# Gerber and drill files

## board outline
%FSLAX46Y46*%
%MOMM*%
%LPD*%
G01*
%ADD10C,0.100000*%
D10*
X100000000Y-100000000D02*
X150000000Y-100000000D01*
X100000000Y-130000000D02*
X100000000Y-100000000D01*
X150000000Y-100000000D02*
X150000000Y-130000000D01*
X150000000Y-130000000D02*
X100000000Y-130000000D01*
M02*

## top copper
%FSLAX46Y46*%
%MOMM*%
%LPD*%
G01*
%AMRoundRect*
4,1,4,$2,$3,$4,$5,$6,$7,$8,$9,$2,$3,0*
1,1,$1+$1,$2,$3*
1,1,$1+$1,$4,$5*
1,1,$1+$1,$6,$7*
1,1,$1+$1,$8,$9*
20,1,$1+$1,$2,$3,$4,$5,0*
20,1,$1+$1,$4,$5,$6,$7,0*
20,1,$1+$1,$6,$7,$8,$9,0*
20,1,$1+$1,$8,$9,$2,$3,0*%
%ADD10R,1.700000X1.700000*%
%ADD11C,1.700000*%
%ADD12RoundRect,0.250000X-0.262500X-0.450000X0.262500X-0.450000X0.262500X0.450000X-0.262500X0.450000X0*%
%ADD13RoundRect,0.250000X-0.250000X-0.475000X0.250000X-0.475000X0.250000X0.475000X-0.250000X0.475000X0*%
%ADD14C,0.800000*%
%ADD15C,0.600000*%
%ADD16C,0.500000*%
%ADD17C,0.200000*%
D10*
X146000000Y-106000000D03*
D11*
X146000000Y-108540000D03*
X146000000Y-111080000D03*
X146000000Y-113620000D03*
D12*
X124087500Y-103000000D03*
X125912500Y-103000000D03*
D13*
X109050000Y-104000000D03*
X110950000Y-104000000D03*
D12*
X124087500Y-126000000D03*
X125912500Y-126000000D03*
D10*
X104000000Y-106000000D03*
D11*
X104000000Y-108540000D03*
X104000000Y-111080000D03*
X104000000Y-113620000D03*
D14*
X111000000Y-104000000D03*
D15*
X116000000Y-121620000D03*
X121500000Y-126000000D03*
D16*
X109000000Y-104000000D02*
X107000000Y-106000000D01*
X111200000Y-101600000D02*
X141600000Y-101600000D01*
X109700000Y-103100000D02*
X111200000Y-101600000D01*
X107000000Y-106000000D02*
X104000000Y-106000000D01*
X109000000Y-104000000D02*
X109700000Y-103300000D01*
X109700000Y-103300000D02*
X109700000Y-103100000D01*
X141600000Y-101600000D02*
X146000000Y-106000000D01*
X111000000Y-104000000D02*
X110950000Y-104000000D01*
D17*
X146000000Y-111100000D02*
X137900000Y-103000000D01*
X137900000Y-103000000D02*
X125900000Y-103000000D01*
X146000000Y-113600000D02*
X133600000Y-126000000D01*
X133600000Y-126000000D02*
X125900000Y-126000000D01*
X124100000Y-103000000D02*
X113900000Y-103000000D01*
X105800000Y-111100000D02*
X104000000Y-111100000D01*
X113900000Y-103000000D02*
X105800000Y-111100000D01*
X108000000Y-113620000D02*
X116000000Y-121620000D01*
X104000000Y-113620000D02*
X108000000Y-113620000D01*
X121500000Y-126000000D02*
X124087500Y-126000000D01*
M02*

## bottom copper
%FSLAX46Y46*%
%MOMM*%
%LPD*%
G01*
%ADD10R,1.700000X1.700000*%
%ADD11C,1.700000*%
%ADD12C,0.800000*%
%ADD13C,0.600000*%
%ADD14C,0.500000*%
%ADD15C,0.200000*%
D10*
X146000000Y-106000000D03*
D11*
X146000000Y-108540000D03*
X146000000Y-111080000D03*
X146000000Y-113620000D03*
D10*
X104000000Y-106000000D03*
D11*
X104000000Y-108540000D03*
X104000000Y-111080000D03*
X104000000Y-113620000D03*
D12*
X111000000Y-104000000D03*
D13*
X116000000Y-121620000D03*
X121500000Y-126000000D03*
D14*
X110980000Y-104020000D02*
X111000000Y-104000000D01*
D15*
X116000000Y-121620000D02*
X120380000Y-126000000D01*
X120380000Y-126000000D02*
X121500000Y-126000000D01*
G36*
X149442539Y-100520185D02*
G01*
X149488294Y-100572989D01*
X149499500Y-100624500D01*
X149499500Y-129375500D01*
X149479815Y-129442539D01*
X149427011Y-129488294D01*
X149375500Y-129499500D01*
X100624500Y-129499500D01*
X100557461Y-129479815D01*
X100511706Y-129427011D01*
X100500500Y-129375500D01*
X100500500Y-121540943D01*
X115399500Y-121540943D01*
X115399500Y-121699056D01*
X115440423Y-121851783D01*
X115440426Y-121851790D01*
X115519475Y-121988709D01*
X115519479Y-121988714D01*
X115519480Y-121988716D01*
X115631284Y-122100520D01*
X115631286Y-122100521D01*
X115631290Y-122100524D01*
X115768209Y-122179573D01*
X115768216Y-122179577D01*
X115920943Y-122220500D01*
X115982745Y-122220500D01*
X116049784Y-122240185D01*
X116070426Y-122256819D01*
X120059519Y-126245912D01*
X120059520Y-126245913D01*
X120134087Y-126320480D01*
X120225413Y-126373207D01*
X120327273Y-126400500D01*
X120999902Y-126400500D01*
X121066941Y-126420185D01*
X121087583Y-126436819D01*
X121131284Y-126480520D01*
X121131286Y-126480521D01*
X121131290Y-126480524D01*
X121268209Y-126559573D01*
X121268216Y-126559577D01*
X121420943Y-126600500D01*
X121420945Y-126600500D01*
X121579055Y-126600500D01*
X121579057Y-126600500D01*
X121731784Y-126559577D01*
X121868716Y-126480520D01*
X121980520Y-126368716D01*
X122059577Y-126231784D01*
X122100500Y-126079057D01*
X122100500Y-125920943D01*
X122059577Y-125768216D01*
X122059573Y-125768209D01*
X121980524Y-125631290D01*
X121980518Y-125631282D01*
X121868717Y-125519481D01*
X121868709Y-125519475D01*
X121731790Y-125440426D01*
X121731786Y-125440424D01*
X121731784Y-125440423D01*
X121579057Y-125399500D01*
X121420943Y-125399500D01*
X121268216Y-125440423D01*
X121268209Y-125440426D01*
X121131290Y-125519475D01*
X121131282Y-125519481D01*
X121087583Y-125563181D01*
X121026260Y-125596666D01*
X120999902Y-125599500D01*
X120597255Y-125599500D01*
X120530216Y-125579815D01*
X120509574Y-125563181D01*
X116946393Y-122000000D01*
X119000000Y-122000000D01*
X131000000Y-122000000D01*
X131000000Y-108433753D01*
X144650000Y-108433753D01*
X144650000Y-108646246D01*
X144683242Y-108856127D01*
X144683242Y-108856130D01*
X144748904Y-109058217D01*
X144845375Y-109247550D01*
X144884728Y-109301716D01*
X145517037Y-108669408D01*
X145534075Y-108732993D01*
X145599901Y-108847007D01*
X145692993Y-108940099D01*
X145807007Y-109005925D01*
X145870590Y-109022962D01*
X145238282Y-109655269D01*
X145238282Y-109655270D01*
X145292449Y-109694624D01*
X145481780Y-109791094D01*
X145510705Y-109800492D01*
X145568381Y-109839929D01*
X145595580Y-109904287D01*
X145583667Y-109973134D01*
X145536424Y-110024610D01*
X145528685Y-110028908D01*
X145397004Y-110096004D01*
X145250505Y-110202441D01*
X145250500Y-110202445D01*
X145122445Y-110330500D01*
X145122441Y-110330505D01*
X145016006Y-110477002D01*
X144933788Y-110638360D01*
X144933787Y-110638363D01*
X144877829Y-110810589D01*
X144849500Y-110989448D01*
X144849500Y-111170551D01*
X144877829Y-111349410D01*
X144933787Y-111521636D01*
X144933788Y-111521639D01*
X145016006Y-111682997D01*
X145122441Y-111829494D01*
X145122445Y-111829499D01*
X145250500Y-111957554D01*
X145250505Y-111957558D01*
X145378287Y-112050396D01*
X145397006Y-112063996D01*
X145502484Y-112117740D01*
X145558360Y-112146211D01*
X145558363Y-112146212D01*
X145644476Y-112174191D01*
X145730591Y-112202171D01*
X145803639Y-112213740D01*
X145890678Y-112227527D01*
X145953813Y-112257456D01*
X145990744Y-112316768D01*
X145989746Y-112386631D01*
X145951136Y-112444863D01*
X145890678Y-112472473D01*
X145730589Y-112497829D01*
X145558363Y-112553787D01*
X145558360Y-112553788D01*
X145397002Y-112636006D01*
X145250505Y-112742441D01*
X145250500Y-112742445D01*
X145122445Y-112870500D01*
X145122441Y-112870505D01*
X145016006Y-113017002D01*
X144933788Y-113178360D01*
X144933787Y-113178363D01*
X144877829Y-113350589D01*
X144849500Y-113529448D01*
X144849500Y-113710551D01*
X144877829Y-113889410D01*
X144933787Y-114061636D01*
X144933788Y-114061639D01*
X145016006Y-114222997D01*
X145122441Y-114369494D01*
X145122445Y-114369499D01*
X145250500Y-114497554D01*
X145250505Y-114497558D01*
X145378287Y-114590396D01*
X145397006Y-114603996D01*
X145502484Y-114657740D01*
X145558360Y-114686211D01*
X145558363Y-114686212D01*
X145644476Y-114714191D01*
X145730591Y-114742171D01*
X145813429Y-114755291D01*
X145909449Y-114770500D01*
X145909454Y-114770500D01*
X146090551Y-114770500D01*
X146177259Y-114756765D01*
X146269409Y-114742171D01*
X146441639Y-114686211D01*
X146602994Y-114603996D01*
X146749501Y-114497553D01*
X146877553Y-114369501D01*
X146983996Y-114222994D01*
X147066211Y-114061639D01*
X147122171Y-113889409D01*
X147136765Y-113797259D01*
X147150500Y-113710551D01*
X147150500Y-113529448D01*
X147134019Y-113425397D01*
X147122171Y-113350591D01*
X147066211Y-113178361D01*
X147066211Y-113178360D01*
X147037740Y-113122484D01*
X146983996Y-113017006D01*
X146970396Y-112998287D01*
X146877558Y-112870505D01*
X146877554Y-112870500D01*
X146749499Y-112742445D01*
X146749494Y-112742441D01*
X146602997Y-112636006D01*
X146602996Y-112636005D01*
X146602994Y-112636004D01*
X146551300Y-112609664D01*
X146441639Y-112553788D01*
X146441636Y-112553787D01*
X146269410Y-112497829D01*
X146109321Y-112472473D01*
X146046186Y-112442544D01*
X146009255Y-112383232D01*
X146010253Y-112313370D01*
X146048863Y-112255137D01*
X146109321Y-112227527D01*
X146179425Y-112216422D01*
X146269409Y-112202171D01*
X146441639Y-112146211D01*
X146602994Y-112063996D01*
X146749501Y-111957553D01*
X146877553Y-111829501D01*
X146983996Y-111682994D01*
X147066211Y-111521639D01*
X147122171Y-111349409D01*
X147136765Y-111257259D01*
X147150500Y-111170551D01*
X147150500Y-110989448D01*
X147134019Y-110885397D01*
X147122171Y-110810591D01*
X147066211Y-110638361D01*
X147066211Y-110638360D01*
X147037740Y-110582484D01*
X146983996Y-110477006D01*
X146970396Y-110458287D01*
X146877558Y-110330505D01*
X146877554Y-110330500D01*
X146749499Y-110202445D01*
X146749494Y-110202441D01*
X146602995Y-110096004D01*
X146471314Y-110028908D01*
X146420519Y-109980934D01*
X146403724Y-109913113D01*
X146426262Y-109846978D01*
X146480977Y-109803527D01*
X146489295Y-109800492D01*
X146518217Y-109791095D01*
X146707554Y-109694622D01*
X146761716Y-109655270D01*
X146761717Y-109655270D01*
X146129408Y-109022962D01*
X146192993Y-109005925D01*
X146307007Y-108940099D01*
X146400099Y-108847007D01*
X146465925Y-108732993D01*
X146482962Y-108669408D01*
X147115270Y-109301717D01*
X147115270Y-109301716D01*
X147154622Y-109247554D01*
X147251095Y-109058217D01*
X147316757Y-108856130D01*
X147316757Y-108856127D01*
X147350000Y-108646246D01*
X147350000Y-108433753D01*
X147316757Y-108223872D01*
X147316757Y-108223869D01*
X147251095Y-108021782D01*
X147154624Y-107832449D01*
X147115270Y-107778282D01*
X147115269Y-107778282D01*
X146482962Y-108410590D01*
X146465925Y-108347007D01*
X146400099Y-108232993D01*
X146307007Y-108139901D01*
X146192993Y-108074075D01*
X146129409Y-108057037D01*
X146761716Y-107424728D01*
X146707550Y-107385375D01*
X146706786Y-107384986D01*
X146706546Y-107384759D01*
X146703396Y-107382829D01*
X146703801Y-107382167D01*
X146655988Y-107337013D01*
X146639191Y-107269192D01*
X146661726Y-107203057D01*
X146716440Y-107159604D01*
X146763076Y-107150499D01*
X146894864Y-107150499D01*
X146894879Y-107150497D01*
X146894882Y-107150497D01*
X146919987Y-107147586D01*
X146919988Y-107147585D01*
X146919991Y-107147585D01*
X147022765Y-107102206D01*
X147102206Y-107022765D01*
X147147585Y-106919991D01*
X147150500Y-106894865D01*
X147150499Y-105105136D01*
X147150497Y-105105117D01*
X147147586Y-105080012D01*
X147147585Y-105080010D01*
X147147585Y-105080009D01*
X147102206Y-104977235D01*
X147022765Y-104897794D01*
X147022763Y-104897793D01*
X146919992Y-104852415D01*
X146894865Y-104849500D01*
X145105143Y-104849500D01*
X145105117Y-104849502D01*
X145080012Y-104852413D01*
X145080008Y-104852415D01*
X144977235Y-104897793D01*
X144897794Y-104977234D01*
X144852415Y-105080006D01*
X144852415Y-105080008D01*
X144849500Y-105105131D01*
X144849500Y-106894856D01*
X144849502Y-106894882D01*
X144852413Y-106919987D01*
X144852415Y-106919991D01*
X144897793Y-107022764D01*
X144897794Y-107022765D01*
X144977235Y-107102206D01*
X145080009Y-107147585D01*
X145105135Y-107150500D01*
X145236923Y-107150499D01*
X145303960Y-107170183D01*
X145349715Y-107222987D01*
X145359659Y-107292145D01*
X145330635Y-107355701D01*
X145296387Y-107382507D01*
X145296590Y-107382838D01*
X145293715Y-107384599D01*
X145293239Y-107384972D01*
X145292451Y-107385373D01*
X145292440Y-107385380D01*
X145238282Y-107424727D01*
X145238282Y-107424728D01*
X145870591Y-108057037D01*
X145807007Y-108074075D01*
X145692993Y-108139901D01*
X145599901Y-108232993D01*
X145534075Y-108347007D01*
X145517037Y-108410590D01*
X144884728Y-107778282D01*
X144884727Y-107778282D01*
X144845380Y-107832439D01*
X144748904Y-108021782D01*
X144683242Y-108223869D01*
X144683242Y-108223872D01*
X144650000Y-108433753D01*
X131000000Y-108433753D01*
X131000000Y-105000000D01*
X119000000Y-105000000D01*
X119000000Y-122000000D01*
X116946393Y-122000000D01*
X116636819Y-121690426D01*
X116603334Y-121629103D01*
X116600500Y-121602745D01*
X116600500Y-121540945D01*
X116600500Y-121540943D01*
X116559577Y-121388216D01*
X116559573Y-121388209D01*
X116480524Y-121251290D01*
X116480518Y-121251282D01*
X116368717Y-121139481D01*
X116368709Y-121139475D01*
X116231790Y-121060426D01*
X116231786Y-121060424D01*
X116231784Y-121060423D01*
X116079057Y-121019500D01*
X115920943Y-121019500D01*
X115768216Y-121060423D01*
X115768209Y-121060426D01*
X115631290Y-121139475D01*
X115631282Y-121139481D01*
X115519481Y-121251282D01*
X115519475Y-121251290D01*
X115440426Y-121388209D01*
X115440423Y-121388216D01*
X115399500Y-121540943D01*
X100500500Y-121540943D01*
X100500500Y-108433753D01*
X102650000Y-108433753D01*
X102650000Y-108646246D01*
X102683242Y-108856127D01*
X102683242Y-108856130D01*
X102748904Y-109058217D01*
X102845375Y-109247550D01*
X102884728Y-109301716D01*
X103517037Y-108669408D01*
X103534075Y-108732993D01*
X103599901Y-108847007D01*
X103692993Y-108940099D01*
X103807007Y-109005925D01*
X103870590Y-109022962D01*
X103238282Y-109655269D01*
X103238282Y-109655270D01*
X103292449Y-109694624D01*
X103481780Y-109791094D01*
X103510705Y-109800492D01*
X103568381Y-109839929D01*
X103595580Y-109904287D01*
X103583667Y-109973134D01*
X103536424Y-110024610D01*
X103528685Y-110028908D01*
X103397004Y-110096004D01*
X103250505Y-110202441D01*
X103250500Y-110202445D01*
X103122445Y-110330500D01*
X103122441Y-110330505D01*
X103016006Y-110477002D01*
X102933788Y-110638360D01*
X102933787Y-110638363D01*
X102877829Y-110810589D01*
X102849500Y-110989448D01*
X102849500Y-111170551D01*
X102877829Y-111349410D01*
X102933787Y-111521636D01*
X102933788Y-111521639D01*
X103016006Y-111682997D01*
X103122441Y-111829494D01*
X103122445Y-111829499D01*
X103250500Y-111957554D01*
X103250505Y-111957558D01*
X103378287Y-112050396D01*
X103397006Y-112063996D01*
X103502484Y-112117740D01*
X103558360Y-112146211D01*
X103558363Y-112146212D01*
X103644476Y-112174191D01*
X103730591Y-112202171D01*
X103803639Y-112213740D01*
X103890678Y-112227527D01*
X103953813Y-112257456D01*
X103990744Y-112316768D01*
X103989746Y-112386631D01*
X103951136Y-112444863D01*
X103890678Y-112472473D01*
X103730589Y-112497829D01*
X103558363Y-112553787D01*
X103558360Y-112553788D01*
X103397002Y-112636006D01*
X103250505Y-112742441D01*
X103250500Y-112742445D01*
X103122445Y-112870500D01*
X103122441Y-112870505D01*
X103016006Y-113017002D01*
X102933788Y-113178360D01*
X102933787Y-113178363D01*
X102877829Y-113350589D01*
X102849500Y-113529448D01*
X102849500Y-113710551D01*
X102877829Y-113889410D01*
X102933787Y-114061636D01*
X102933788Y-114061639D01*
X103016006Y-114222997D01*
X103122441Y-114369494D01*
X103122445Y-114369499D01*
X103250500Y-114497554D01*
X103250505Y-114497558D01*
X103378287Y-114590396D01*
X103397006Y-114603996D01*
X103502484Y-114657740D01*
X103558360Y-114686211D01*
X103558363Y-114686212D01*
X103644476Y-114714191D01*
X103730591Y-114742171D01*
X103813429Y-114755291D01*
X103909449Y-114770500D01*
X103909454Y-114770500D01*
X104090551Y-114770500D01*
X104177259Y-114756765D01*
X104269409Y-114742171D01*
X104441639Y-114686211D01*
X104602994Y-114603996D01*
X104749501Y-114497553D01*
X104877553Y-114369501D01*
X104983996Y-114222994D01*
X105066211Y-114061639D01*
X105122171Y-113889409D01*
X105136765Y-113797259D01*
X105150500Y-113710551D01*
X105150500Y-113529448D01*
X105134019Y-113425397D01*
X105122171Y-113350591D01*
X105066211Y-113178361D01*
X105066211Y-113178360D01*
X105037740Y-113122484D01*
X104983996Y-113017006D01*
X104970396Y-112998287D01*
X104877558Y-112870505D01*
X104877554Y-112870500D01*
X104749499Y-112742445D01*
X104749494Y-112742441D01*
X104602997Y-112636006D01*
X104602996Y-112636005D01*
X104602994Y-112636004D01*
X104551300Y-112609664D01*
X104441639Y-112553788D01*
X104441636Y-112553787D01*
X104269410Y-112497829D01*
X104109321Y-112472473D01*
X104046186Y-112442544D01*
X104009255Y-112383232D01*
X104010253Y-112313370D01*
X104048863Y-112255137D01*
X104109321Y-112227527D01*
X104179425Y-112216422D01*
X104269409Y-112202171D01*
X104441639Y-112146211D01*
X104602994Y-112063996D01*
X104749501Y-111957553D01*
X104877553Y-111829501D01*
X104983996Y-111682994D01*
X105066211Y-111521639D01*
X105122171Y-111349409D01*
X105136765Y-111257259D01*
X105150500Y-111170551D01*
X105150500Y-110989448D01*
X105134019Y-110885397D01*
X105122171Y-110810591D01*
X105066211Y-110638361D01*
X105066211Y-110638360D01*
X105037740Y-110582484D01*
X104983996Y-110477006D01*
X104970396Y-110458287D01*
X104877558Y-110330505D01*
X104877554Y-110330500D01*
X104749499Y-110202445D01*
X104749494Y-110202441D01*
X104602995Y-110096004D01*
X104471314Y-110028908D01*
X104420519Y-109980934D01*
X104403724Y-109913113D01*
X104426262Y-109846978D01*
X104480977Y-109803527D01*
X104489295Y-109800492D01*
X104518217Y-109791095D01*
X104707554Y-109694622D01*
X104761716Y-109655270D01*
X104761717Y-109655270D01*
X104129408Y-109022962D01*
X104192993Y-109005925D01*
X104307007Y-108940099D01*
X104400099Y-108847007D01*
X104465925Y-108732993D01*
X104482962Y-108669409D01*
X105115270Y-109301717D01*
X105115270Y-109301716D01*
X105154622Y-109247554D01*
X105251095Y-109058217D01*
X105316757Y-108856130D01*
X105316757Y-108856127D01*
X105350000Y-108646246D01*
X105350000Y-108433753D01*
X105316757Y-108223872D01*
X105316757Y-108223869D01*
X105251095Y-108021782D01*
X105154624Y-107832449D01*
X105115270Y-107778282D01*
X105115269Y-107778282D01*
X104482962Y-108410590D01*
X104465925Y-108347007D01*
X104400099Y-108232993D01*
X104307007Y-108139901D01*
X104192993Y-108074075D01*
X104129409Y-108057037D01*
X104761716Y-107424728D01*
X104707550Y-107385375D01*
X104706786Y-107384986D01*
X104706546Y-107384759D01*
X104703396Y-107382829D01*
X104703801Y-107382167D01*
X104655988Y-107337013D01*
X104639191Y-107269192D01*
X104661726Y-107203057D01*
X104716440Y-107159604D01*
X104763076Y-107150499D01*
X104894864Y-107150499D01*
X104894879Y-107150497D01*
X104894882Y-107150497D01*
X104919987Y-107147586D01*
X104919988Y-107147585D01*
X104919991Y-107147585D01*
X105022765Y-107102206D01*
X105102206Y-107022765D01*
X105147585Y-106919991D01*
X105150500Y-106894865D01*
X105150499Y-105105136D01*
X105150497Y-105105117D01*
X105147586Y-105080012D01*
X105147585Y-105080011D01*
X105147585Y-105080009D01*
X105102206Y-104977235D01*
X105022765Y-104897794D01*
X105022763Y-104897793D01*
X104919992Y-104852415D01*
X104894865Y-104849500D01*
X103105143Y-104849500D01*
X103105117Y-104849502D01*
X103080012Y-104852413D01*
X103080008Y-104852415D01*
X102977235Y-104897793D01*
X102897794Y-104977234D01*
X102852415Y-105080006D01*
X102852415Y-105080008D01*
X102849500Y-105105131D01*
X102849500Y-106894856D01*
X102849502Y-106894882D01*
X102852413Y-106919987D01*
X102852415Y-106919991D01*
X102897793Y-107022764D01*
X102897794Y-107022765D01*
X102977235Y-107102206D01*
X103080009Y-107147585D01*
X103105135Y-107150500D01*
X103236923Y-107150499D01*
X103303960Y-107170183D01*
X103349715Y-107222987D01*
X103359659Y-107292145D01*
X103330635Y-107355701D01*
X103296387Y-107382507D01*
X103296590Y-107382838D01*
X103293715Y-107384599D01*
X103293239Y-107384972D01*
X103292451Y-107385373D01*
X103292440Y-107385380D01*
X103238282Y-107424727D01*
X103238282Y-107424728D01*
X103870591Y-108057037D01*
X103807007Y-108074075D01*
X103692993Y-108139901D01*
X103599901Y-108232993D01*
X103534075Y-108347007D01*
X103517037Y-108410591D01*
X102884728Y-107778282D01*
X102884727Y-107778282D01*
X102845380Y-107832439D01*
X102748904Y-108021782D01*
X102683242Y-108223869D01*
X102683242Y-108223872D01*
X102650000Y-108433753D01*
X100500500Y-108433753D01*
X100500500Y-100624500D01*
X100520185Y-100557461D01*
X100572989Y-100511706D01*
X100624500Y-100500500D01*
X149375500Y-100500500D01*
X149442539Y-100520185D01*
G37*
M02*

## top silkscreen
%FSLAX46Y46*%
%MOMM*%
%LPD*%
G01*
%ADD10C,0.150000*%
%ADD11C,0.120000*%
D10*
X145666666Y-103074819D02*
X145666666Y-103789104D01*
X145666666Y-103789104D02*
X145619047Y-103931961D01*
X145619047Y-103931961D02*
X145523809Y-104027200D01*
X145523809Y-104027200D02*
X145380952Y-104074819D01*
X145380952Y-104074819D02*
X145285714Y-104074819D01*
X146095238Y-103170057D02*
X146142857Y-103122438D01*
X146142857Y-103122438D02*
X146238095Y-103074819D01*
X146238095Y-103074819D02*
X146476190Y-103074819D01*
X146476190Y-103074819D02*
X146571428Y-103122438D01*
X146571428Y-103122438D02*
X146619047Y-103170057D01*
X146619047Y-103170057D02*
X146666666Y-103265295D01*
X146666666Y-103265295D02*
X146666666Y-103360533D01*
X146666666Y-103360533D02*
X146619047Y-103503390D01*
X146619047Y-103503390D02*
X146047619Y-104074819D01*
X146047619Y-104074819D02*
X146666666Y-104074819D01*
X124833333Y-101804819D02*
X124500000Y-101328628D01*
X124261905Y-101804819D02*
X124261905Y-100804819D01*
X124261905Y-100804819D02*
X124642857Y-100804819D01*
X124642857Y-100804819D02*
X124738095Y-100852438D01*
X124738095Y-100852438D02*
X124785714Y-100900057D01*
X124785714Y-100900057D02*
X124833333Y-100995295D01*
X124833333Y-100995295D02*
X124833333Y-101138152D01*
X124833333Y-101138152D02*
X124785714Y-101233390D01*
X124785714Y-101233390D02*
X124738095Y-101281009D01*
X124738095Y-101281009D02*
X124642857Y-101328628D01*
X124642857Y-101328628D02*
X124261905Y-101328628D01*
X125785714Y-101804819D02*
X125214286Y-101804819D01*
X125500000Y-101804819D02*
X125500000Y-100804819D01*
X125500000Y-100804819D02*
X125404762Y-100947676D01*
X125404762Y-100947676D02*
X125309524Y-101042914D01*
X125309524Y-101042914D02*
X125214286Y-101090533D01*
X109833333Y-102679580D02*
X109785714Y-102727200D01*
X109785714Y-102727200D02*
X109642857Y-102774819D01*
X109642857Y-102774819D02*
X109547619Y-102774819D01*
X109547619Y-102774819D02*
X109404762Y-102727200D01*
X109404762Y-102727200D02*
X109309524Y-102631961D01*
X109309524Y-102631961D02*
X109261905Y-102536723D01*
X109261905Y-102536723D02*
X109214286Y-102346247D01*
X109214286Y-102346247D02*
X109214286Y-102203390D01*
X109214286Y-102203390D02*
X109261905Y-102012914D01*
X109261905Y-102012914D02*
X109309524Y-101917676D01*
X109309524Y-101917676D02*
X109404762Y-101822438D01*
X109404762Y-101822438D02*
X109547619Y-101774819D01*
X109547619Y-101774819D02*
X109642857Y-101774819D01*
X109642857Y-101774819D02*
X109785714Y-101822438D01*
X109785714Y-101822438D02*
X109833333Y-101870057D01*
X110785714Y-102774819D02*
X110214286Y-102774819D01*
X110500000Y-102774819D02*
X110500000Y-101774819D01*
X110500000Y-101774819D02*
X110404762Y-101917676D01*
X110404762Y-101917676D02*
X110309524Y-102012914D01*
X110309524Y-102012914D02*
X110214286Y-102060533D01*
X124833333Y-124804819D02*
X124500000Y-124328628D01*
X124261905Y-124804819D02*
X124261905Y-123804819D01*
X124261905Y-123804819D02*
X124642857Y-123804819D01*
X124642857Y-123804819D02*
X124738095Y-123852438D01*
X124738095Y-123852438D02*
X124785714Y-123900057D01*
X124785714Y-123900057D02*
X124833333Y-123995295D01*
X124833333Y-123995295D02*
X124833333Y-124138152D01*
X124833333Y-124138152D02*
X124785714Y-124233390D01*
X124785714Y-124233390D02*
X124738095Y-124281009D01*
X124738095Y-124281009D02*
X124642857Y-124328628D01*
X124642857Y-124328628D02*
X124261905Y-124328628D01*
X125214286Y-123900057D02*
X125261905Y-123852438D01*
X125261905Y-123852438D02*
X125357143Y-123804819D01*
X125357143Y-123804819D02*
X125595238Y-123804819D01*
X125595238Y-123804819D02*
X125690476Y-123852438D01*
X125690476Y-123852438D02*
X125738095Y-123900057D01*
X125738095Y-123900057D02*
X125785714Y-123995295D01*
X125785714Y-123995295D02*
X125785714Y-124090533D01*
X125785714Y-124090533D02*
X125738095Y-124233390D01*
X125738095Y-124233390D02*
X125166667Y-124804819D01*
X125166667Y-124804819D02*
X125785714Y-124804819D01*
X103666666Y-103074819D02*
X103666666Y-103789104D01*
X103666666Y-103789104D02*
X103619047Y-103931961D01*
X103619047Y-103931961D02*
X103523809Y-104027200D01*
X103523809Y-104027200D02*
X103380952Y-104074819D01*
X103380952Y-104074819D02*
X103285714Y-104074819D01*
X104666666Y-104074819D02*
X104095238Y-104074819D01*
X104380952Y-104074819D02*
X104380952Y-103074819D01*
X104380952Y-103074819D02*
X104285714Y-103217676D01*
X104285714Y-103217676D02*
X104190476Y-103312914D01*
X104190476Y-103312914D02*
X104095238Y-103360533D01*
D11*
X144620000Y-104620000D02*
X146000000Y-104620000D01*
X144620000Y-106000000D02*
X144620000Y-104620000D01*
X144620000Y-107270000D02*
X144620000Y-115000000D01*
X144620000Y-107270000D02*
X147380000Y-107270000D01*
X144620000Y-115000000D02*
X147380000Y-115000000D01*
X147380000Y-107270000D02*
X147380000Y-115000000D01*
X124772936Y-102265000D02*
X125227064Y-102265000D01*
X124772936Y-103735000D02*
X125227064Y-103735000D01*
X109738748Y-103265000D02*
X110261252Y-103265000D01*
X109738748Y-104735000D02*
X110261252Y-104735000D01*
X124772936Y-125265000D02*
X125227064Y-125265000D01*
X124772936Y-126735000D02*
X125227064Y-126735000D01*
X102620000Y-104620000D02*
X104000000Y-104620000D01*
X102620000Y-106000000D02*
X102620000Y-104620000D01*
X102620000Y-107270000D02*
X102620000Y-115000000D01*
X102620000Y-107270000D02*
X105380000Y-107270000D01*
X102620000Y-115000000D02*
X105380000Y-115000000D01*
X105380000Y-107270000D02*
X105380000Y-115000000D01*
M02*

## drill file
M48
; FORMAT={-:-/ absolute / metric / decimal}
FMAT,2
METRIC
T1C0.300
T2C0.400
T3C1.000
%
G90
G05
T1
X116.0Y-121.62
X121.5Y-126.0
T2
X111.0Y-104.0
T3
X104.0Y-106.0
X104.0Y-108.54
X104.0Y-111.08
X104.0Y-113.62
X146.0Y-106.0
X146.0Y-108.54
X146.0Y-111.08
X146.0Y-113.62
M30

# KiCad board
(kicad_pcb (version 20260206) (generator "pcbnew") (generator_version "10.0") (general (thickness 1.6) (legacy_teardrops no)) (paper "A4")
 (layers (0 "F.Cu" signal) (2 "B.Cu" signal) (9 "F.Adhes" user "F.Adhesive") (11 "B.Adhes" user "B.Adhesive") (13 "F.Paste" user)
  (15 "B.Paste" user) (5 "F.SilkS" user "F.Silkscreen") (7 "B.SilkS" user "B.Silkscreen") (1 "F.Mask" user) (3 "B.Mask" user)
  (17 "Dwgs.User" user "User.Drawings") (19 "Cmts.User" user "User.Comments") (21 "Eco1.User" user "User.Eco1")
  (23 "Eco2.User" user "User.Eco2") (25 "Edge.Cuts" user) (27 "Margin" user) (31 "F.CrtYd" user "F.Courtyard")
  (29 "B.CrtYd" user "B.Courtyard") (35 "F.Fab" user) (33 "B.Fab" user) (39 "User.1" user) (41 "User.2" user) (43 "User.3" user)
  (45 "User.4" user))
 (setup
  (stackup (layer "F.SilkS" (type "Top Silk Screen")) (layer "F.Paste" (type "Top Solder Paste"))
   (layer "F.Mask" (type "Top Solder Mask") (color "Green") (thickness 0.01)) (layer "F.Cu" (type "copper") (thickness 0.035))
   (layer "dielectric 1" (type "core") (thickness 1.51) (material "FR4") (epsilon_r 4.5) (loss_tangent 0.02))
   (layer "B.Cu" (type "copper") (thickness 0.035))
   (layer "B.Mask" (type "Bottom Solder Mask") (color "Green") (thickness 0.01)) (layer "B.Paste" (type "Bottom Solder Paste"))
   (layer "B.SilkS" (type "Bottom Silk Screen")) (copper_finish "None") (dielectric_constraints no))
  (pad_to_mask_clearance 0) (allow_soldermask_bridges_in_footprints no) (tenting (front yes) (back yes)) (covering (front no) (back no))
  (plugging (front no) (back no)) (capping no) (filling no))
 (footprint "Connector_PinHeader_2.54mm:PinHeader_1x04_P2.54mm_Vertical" (layer "F.Cu") (at 146 106)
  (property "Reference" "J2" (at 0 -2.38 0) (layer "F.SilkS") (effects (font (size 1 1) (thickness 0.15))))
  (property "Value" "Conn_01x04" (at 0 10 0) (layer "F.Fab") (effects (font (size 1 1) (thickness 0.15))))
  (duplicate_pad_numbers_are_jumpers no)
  (fp_line (start -1.38 -1.38) (end 0 -1.38) (stroke (width 0.12) (type solid)) (layer "F.SilkS"))
  (fp_line (start -1.38 0) (end -1.38 -1.38) (stroke (width 0.12) (type solid)) (layer "F.SilkS"))
  (fp_line (start -1.38 1.27) (end -1.38 9) (stroke (width 0.12) (type solid)) (layer "F.SilkS"))
  (fp_line (start -1.38 1.27) (end 1.38 1.27) (stroke (width 0.12) (type solid)) (layer "F.SilkS"))
  (fp_line (start -1.38 9) (end 1.38 9) (stroke (width 0.12) (type solid)) (layer "F.SilkS"))
  (fp_line (start 1.38 1.27) (end 1.38 9) (stroke (width 0.12) (type solid)) (layer "F.SilkS"))
  (pad "1" thru_hole rect (at 0 0) (size 1.7 1.7) (drill 1) (layers "*.Cu" "*.Mask") (remove_unused_layers no) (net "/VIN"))
  (pad "2" thru_hole circle (at 0 2.54) (size 1.7 1.7) (drill 1) (layers "*.Cu" "*.Mask") (remove_unused_layers no) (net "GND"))
  (pad "3" thru_hole circle (at 0 5.08) (size 1.7 1.7) (drill 1) (layers "*.Cu" "*.Mask") (remove_unused_layers no) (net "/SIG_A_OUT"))
  (pad "4" thru_hole circle (at 0 7.62) (size 1.7 1.7) (drill 1) (layers "*.Cu" "*.Mask") (remove_unused_layers no) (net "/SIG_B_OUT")))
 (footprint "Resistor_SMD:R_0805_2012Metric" (layer "F.Cu") (at 125 103)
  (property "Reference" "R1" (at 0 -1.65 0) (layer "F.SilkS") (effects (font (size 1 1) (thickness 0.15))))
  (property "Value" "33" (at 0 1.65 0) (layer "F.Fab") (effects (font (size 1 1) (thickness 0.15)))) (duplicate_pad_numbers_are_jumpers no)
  (fp_line (start -0.227064 -0.735) (end 0.227064 -0.735) (stroke (width 0.12) (type solid)) (layer "F.SilkS"))
  (fp_line (start -0.227064 0.735) (end 0.227064 0.735) (stroke (width 0.12) (type solid)) (layer "F.SilkS"))
  (pad "1" smd roundrect (at -0.9125 0) (size 1.025 1.4) (layers "F.Cu" "F.Mask" "F.Paste") (roundrect_rratio 0.243902) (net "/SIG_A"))
  (pad "2" smd roundrect (at 0.9125 0) (size 1.025 1.4) (layers "F.Cu" "F.Mask" "F.Paste") (roundrect_rratio 0.243902) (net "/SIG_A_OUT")))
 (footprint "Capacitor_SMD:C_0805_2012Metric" (layer "F.Cu") (at 110 104)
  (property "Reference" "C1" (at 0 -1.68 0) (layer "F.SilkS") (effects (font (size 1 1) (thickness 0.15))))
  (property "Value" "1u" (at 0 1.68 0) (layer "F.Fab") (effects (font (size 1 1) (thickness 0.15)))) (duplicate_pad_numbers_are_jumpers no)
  (fp_line (start -0.261252 -0.735) (end 0.261252 -0.735) (stroke (width 0.12) (type solid)) (layer "F.SilkS"))
  (fp_line (start -0.261252 0.735) (end 0.261252 0.735) (stroke (width 0.12) (type solid)) (layer "F.SilkS"))
  (pad "1" smd roundrect (at -0.95 0) (size 1 1.45) (layers "F.Cu" "F.Mask" "F.Paste") (roundrect_rratio 0.25) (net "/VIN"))
  (pad "2" smd roundrect (at 0.95 0) (size 1 1.45) (layers "F.Cu" "F.Mask" "F.Paste") (roundrect_rratio 0.25) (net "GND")))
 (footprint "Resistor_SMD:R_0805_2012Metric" (layer "F.Cu") (at 125 126)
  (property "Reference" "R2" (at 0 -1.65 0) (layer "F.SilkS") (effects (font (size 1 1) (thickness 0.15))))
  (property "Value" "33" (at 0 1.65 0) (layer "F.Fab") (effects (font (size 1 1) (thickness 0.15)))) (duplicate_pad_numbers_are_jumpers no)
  (fp_line (start -0.227064 -0.735) (end 0.227064 -0.735) (stroke (width 0.12) (type solid)) (layer "F.SilkS"))
  (fp_line (start -0.227064 0.735) (end 0.227064 0.735) (stroke (width 0.12) (type solid)) (layer "F.SilkS"))
  (pad "1" smd roundrect (at -0.9125 0) (size 1.025 1.4) (layers "F.Cu" "F.Mask" "F.Paste") (roundrect_rratio 0.243902) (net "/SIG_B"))
  (pad "2" smd roundrect (at 0.9125 0) (size 1.025 1.4) (layers "F.Cu" "F.Mask" "F.Paste") (roundrect_rratio 0.243902) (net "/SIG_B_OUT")))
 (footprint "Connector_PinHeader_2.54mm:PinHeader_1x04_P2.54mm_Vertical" (layer "F.Cu") (at 104 106)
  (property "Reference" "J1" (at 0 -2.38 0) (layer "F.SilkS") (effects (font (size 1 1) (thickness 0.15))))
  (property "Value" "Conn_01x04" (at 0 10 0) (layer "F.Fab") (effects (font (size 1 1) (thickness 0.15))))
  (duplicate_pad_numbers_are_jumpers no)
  (fp_line (start -1.38 -1.38) (end 0 -1.38) (stroke (width 0.12) (type solid)) (layer "F.SilkS"))
  (fp_line (start -1.38 0) (end -1.38 -1.38) (stroke (width 0.12) (type solid)) (layer "F.SilkS"))
  (fp_line (start -1.38 1.27) (end -1.38 9) (stroke (width 0.12) (type solid)) (layer "F.SilkS"))
  (fp_line (start -1.38 1.27) (end 1.38 1.27) (stroke (width 0.12) (type solid)) (layer "F.SilkS"))
  (fp_line (start -1.38 9) (end 1.38 9) (stroke (width 0.12) (type solid)) (layer "F.SilkS"))
  (fp_line (start 1.38 1.27) (end 1.38 9) (stroke (width 0.12) (type solid)) (layer "F.SilkS"))
  (pad "1" thru_hole rect (at 0 0) (size 1.7 1.7) (drill 1) (layers "*.Cu" "*.Mask") (remove_unused_layers no) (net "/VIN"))
  (pad "2" thru_hole circle (at 0 2.54) (size 1.7 1.7) (drill 1) (layers "*.Cu" "*.Mask") (remove_unused_layers no) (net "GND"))
  (pad "3" thru_hole circle (at 0 5.08) (size 1.7 1.7) (drill 1) (layers "*.Cu" "*.Mask") (remove_unused_layers no) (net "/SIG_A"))
  (pad "4" thru_hole circle (at 0 7.62) (size 1.7 1.7) (drill 1) (layers "*.Cu" "*.Mask") (remove_unused_layers no) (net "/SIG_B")))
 (gr_line (start 100 100) (end 150 100) (stroke (width 0.1) (type default)) (layer "Edge.Cuts"))
 (gr_line (start 100 130) (end 100 100) (stroke (width 0.1) (type default)) (layer "Edge.Cuts"))
 (gr_line (start 150 100) (end 150 130) (stroke (width 0.1) (type default)) (layer "Edge.Cuts"))
 (gr_line (start 150 130) (end 100 130) (stroke (width 0.1) (type default)) (layer "Edge.Cuts"))
 (segment (start 109 104) (end 107 106) (width 0.5) (layer "F.Cu") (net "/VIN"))
 (segment (start 111.2 101.6) (end 141.6 101.6) (width 0.5) (layer "F.Cu") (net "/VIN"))
 (segment (start 109.7 103.1) (end 111.2 101.6) (width 0.5) (layer "F.Cu") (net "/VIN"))
 (segment (start 107 106) (end 104 106) (width 0.5) (layer "F.Cu") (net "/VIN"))
 (segment (start 109 104) (end 109.7 103.3) (width 0.5) (layer "F.Cu") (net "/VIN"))
 (segment (start 109.7 103.3) (end 109.7 103.1) (width 0.5) (layer "F.Cu") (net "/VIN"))
 (segment (start 141.6 101.6) (end 146 106) (width 0.5) (layer "F.Cu") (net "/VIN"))
 (segment (start 111 104) (end 110.95 104) (width 0.5) (layer "F.Cu") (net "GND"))
 (via (at 111 104) (size 0.8) (drill 0.4) (layers "F.Cu" "B.Cu") (capping yes) (filling yes) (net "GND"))
 (segment (start 110.98 104.02) (end 111 104) (width 0.5) (layer "B.Cu") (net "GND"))
 (segment (start 146 111.1) (end 137.9 103) (width 0.2) (layer "F.Cu") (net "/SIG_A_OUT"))
 (segment (start 137.9 103) (end 125.9 103) (width 0.2) (layer "F.Cu") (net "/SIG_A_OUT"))
 (segment (start 146 113.6) (end 133.6 126) (width 0.2) (layer "F.Cu") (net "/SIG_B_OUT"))
 (segment (start 133.6 126) (end 125.9 126) (width 0.2) (layer "F.Cu") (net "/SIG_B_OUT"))
 (segment (start 124.1 103) (end 113.9 103) (width 0.2) (layer "F.Cu") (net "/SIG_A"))
 (segment (start 105.8 111.1) (end 104 111.1) (width 0.2) (layer "F.Cu") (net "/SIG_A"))
 (segment (start 113.9 103) (end 105.8 111.1) (width 0.2) (layer "F.Cu") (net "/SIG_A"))
 (segment (start 108 113.62) (end 116 121.62) (width 0.2) (locked yes) (layer "F.Cu") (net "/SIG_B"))
 (segment (start 104 113.62) (end 108 113.62) (width 0.2) (locked yes) (layer "F.Cu") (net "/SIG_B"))
 (segment (start 121.5 126) (end 124.0875 126) (width 0.2) (locked yes) (layer "F.Cu") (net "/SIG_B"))
 (via (at 116 121.62) (size 0.6) (drill 0.3) (layers "F.Cu" "B.Cu") (locked yes) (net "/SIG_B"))
 (via (at 121.5 126) (size 0.6) (drill 0.3) (layers "F.Cu" "B.Cu") (locked yes) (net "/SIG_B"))
 (segment (start 116 121.62) (end 120.38 126) (width 0.2) (locked yes) (layer "B.Cu") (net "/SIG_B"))
 (segment (start 120.38 126) (end 121.5 126) (width 0.2) (locked yes) (layer "B.Cu") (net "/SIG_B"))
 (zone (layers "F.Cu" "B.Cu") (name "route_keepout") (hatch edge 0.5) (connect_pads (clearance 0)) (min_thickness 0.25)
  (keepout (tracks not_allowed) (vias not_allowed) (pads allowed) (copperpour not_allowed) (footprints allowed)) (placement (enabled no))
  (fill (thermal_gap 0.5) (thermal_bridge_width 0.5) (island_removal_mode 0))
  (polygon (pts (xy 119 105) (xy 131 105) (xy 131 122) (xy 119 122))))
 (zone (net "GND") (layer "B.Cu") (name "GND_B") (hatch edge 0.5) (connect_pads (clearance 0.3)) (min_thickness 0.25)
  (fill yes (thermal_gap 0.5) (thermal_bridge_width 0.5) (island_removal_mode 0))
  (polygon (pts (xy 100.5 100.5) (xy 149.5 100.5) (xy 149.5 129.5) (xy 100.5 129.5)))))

